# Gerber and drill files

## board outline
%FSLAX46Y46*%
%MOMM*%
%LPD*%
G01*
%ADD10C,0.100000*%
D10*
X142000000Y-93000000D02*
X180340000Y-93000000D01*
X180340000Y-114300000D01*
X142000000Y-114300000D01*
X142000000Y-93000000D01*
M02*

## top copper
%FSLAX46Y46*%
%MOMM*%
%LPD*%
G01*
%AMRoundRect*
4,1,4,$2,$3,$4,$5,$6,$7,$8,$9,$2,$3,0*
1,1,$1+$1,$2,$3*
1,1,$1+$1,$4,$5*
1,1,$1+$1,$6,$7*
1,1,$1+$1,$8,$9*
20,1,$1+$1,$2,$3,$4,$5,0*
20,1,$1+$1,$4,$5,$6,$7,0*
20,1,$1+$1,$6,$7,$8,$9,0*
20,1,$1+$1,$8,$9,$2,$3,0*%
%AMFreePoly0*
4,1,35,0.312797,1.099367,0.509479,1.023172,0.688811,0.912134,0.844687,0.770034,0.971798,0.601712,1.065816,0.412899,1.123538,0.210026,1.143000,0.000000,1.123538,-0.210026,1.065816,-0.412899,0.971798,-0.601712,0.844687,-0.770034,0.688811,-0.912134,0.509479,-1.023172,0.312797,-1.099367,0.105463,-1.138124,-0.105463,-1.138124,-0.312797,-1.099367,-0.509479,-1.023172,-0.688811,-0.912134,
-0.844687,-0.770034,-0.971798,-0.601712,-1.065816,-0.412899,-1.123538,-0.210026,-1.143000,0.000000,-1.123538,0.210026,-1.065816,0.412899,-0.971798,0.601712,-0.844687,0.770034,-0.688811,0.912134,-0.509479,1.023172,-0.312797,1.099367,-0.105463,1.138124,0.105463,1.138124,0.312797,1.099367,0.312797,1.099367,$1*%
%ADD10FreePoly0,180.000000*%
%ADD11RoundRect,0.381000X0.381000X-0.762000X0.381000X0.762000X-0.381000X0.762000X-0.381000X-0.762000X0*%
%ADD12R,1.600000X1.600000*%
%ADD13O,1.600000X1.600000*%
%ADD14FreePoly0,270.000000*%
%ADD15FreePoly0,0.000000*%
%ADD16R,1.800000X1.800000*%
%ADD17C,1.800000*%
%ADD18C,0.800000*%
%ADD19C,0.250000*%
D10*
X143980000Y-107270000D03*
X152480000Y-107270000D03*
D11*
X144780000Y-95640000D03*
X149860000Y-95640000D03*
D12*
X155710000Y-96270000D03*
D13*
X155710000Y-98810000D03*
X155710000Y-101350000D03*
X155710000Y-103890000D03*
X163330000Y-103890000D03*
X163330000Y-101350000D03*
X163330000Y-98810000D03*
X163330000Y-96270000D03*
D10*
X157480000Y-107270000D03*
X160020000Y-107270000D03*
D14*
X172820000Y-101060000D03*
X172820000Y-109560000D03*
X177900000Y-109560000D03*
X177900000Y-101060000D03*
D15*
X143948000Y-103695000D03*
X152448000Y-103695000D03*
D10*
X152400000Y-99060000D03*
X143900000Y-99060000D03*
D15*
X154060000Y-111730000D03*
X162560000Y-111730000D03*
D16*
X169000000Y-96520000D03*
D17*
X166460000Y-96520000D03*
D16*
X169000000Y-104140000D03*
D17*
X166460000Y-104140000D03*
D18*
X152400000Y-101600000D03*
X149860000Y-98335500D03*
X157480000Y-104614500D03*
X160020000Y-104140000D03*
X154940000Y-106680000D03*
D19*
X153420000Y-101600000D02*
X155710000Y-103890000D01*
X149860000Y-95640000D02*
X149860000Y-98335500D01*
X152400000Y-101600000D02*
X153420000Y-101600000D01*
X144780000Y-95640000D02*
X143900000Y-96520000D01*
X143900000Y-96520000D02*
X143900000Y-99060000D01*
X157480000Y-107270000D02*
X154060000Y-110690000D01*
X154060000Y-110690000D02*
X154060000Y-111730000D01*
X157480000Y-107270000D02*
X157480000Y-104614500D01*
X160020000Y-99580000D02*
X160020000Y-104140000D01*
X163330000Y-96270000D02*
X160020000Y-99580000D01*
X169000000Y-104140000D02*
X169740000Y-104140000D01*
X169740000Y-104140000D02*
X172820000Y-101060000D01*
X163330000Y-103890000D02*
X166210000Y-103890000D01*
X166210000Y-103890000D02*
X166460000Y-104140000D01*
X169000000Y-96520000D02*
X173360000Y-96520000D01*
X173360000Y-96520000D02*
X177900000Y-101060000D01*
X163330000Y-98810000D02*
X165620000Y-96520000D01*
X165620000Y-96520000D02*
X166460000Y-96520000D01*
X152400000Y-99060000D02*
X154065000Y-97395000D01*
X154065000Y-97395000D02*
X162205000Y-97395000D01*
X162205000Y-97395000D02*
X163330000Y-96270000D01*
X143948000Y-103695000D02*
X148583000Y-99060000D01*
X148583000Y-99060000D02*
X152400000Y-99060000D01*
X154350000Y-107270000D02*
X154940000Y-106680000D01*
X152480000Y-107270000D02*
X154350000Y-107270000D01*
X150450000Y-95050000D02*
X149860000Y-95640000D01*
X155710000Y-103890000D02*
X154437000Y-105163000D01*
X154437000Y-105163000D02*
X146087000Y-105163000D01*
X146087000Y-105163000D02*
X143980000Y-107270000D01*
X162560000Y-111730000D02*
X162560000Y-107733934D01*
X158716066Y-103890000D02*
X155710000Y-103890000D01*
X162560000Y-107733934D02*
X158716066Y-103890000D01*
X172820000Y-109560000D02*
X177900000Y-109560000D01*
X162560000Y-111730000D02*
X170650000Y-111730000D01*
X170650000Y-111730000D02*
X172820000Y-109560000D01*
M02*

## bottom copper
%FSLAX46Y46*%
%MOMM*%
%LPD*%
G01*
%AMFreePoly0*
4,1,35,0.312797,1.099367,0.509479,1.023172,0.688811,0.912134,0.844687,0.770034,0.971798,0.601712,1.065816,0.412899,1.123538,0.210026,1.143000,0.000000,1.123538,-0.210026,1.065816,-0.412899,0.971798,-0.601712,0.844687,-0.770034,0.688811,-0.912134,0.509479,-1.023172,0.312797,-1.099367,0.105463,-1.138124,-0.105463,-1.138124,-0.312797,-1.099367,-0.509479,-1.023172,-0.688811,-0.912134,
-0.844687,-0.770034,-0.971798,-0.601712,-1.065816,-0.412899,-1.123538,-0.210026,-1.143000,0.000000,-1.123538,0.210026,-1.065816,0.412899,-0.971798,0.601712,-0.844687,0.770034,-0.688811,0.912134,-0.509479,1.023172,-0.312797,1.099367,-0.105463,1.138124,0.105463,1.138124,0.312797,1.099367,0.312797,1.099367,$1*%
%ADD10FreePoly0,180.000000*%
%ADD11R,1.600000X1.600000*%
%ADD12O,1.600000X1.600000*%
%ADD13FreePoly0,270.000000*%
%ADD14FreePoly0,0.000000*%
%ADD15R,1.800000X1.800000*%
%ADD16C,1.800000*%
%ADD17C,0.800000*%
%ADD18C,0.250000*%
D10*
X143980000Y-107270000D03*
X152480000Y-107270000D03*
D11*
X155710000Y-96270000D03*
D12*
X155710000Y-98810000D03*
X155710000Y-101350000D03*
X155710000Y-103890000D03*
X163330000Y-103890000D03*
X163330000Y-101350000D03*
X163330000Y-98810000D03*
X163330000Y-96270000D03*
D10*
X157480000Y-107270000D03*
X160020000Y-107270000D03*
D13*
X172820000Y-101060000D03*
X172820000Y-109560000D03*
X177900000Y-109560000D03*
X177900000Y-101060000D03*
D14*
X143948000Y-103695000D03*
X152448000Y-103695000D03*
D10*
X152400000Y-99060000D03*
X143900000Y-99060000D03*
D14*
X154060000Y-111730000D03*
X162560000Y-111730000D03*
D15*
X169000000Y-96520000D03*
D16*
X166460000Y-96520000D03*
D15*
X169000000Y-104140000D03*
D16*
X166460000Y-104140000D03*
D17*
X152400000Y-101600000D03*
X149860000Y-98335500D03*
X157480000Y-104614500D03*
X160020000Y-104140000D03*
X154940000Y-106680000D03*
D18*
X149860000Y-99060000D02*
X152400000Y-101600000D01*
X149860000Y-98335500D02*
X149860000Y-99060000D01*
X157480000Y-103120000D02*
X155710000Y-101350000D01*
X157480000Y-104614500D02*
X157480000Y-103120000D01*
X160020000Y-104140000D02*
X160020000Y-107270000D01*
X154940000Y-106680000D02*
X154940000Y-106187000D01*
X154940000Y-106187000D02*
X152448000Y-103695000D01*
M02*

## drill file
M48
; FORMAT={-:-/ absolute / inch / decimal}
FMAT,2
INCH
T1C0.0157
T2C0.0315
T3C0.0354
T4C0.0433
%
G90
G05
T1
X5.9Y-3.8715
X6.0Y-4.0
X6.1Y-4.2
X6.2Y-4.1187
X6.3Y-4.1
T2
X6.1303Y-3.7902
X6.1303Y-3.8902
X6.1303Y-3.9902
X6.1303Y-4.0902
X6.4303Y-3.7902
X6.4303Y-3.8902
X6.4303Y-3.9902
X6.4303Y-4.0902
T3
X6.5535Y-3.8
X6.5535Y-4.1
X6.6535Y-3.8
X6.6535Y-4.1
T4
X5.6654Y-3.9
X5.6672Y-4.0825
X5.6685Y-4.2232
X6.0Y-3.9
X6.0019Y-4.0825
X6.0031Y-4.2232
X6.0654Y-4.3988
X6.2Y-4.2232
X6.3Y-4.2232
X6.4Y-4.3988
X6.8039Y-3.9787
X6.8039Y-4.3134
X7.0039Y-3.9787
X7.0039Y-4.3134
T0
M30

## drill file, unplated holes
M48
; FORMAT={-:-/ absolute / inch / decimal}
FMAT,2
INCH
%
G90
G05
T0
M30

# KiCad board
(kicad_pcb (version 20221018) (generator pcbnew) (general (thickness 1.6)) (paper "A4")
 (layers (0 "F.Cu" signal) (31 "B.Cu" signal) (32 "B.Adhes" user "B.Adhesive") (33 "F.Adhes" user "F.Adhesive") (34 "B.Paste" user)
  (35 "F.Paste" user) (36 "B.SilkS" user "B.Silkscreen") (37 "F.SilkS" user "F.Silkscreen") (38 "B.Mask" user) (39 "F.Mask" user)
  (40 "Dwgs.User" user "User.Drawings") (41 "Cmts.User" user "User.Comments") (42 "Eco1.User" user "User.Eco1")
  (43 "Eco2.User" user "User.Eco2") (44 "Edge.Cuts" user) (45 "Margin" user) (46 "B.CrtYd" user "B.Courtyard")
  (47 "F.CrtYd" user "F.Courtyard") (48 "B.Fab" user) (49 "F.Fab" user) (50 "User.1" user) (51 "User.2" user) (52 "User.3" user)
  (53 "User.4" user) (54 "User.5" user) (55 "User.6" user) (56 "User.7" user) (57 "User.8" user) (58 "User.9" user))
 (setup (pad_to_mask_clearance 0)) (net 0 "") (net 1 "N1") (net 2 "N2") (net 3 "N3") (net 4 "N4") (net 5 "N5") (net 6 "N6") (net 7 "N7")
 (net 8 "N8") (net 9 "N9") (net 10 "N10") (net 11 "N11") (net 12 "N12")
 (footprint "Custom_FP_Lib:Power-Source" (layer "F.Cu") (at 147.32 98.18 90)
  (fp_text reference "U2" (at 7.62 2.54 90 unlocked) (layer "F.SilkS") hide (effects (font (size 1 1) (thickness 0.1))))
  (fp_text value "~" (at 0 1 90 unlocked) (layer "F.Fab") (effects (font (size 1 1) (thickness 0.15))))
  (pad "1" smd roundrect (at 2.54 -2.54 90) (size 2.286 1.524) (layers "F.Cu" "F.Paste" "F.Mask") (roundrect_rratio 0.25) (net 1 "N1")
   (thermal_bridge_angle 45))
  (pad "2" smd roundrect (at 2.54 2.54 90) (size 2.286 1.524) (layers "F.Cu" "F.Paste" "F.Mask") (roundrect_rratio 0.25) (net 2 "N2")
   (thermal_bridge_angle 45)))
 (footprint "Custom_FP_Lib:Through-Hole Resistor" (layer "F.Cu") (at 143.628 104.965)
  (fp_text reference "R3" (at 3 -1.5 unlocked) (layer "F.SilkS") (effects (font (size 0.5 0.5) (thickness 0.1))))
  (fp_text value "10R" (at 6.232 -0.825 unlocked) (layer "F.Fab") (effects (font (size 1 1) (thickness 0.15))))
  (pad "1" thru_hole custom (at 0.32 -1.27) (size 2.286 2.286) (drill 1.1) (layers "*.Cu" "*.Mask") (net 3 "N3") (thermal_bridge_angle 45)
   (options (clearance outline) (anchor circle)) (primitives))
  (pad "2" thru_hole custom (at 8.82 -1.27) (size 2.286 2.286) (drill 1.1) (layers "*.Cu" "*.Mask") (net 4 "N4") (thermal_bridge_angle 45)
   (options (clearance outline) (anchor circle)) (primitives)))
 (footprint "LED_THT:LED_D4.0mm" (layer "F.Cu") (at 169 104.14 180)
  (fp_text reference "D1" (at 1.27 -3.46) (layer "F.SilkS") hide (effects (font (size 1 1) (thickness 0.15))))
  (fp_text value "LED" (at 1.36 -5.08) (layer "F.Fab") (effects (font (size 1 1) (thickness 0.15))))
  (pad "1" thru_hole rect (at 0 0 180) (size 1.8 1.8) (drill 0.9) (layers "*.Cu" "*.Mask") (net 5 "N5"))
  (pad "2" thru_hole circle (at 2.54 0 180) (size 1.8 1.8) (drill 0.9) (layers "*.Cu" "*.Mask") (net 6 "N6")))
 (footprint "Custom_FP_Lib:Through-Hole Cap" (layer "F.Cu") (at 160.02 106 180)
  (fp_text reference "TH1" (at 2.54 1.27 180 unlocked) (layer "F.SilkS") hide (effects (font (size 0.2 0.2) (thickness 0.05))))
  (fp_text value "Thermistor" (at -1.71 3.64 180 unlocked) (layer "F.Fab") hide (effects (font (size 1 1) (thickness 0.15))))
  (pad "1" thru_hole custom (at 0 -1.27 180) (size 2.286 2.286) (drill 1.1) (layers "*.Cu" "*.Mask") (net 3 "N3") (thermal_bridge_angle 45)
   (options (clearance outline) (anchor circle)) (primitives))
  (pad "2" thru_hole custom (at 2.54 -1.27 180) (size 2.286 2.286) (drill 1.1) (layers "*.Cu" "*.Mask") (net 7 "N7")
   (thermal_bridge_angle 45) (options (clearance outline) (anchor circle)) (primitives)))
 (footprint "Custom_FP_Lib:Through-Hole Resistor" (layer "F.Cu") (at 176.63 100.74 -90)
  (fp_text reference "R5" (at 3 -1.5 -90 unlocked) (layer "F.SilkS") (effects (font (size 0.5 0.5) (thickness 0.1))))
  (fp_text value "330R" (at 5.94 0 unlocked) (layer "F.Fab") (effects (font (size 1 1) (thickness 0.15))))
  (pad "1" thru_hole custom (at 0.32 -1.27 270) (size 2.286 2.286) (drill 1.1) (layers "*.Cu" "*.Mask") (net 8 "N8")
   (thermal_bridge_angle 45) (options (clearance outline) (anchor circle)) (primitives))
  (pad "2" thru_hole custom (at 8.82 -1.27 270) (size 2.286 2.286) (drill 1.1) (layers "*.Cu" "*.Mask") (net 2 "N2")
   (thermal_bridge_angle 45) (options (clearance outline) (anchor circle)) (primitives)))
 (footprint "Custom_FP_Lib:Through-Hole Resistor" (layer "F.Cu") (at 152.8 106 180)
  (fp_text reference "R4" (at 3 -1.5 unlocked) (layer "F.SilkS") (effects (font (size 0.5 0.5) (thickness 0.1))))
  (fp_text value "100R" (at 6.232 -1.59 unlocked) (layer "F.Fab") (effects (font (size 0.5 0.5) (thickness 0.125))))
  (pad "1" thru_hole custom (at 0.32 -1.27 180) (size 2.286 2.286) (drill 1.1) (layers "*.Cu" "*.Mask") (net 4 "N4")
   (thermal_bridge_angle 45) (options (clearance outline) (anchor circle)) (primitives))
  (pad "2" thru_hole custom (at 8.82 -1.27 180) (size 2.286 2.286) (drill 1.1) (layers "*.Cu" "*.Mask") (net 2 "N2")
   (thermal_bridge_angle 45) (options (clearance outline) (anchor circle)) (primitives)))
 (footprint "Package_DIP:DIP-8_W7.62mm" (layer "F.Cu") (at 155.71 96.27)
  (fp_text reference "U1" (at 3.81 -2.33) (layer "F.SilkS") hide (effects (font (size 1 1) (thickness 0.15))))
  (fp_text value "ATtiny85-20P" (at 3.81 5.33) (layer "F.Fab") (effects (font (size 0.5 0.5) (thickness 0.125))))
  (pad "1" thru_hole rect (at 0 0) (size 1.6 1.6) (drill 0.8) (layers "*.Cu" "*.Mask") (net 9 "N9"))
  (pad "2" thru_hole oval (at 0 2.54) (size 1.6 1.6) (drill 0.8) (layers "*.Cu" "*.Mask") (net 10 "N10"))
  (pad "3" thru_hole oval (at 0 5.08) (size 1.6 1.6) (drill 0.8) (layers "*.Cu" "*.Mask") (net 7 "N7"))
  (pad "4" thru_hole oval (at 0 7.62) (size 1.6 1.6) (drill 0.8) (layers "*.Cu" "*.Mask") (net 2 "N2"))
  (pad "5" thru_hole oval (at 7.62 7.62) (size 1.6 1.6) (drill 0.8) (layers "*.Cu" "*.Mask") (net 6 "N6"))
  (pad "6" thru_hole oval (at 7.62 5.08) (size 1.6 1.6) (drill 0.8) (layers "*.Cu" "*.Mask") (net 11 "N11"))
  (pad "7" thru_hole oval (at 7.62 2.54) (size 1.6 1.6) (drill 0.8) (layers "*.Cu" "*.Mask") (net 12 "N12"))
  (pad "8" thru_hole oval (at 7.62 0) (size 1.6 1.6) (drill 0.8) (layers "*.Cu" "*.Mask") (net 3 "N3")))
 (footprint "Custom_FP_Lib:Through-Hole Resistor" (layer "F.Cu") (at 152.72 97.79 180)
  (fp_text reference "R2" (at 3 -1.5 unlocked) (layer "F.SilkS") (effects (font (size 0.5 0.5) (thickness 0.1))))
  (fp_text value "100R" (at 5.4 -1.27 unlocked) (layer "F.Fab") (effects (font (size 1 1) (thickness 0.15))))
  (pad "1" thru_hole custom (at 0.32 -1.27 180) (size 2.286 2.286) (drill 1.1) (layers "*.Cu" "*.Mask") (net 3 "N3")
   (thermal_bridge_angle 45) (options (clearance outline) (anchor circle)) (primitives))
  (pad "2" thru_hole custom (at 8.82 -1.27 180) (size 2.286 2.286) (drill 1.1) (layers "*.Cu" "*.Mask") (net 1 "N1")
   (thermal_bridge_angle 45) (options (clearance outline) (anchor circle)) (primitives)))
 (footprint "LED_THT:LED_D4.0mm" (layer "F.Cu") (at 169 96.52 180)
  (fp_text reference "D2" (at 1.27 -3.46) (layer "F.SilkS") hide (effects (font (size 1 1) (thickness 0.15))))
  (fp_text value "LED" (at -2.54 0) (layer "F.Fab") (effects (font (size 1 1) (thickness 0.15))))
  (pad "1" thru_hole rect (at 0 0 180) (size 1.8 1.8) (drill 0.9) (layers "*.Cu" "*.Mask") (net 8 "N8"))
  (pad "2" thru_hole circle (at 2.54 0 180) (size 1.8 1.8) (drill 0.9) (layers "*.Cu" "*.Mask") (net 12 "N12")))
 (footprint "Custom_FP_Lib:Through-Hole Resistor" (layer "F.Cu") (at 171.55 100.74 -90)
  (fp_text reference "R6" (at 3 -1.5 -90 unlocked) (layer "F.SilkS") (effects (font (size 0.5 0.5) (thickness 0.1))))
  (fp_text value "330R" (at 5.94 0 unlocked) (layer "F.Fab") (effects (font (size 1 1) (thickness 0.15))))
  (pad "1" thru_hole custom (at 0.32 -1.27 270) (size 2.286 2.286) (drill 1.1) (layers "*.Cu" "*.Mask") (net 5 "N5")
   (thermal_bridge_angle 45) (options (clearance outline) (anchor circle)) (primitives))
  (pad "2" thru_hole custom (at 8.82 -1.27 270) (size 2.286 2.286) (drill 1.1) (layers "*.Cu" "*.Mask") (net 2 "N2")
   (thermal_bridge_angle 45) (options (clearance outline) (anchor circle)) (primitives)))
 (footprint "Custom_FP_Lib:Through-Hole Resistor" (layer "F.Cu") (at 153.74 113)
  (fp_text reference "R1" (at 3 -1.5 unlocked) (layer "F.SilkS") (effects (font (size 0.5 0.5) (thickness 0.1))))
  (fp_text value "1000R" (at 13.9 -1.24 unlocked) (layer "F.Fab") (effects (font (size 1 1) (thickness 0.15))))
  (pad "1" thru_hole custom (at 0.32 -1.27) (size 2.286 2.286) (drill 1.1) (layers "*.Cu" "*.Mask") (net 7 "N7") (thermal_bridge_angle 45)
   (options (clearance outline) (anchor circle)) (primitives))
  (pad "2" thru_hole custom (at 8.82 -1.27) (size 2.286 2.286) (drill 1.1) (layers "*.Cu" "*.Mask") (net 2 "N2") (thermal_bridge_angle 45)
   (options (clearance outline) (anchor circle)) (primitives)))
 (gr_rect (start 142 93) (end 180.34 114.3) (stroke (width 0.1) (type default)) (fill none) (layer "Edge.Cuts"))
 (segment (start 169.74 104.14) (end 172.82 101.06) (width 0.25) (layer "F.Cu") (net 5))
 (segment (start 169 104.14) (end 169.74 104.14) (width 0.25) (layer "F.Cu") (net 5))
 (segment (start 166.21 103.89) (end 166.46 104.14) (width 0.25) (layer "F.Cu") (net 6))
 (segment (start 163.33 103.89) (end 166.21 103.89) (width 0.25) (layer "F.Cu") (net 6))
 (segment (start 163.33 98.81) (end 165.62 96.52) (width 0.25) (layer "F.Cu") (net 12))
 (segment (start 165.62 96.52) (end 166.46 96.52) (width 0.25) (layer "F.Cu") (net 12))
 (segment (start 154.06 110.69) (end 154.06 111.73) (width 0.25) (layer "F.Cu") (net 7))
 (segment (start 157.48 107.27) (end 154.06 110.69) (width 0.25) (layer "F.Cu") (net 7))
 (segment (start 157.48 107.27) (end 157.48 104.6145) (width 0.25) (layer "F.Cu") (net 7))
 (via (at 157.48 104.6145) (size 0.8) (drill 0.4) (layers "F.Cu" "B.Cu") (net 7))
 (segment (start 157.48 104.6145) (end 157.48 103.12) (width 0.25) (layer "B.Cu") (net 7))
 (segment (start 157.48 103.12) (end 155.71 101.35) (width 0.25) (layer "B.Cu") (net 7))
 (segment (start 162.205 97.395) (end 163.33 96.27) (width 0.25) (layer "F.Cu") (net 3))
 (segment (start 152.4 99.06) (end 154.065 97.395) (width 0.25) (layer "F.Cu") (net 3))
 (segment (start 148.583 99.06) (end 152.4 99.06) (width 0.25) (layer "F.Cu") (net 3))
 (segment (start 160.02 99.58) (end 160.02 104.14) (width 0.25) (layer "F.Cu") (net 3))
 (segment (start 163.33 96.27) (end 160.02 99.58) (width 0.25) (layer "F.Cu") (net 3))
 (segment (start 143.948 103.695) (end 148.583 99.06) (width 0.25) (layer "F.Cu") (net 3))
 (segment (start 154.065 97.395) (end 162.205 97.395) (width 0.25) (layer "F.Cu") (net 3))
 (via (at 160.02 104.14) (size 0.8) (drill 0.4) (layers "F.Cu" "B.Cu") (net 3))
 (segment (start 160.02 104.14) (end 160.02 107.27) (width 0.25) (layer "B.Cu") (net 3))
 (segment (start 143.9 96.52) (end 143.9 99.06) (width 0.25) (layer "F.Cu") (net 1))
 (segment (start 144.78 95.64) (end 143.9 96.52) (width 0.25) (layer "F.Cu") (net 1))
 (segment (start 152.48 107.27) (end 154.35 107.27) (width 0.25) (layer "F.Cu") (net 4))
 (segment (start 154.35 107.27) (end 154.94 106.68) (width 0.25) (layer "F.Cu") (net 4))
 (via (at 154.94 106.68) (size 0.8) (drill 0.4) (layers "F.Cu" "B.Cu") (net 4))
 (segment (start 154.94 106.187) (end 152.448 103.695) (width 0.25) (layer "B.Cu") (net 4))
 (segment (start 154.94 106.68) (end 154.94 106.187) (width 0.25) (layer "B.Cu") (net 4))
 (segment (start 173.36 96.52) (end 177.9 101.06) (width 0.25) (layer "F.Cu") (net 8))
 (segment (start 169 96.52) (end 173.36 96.52) (width 0.25) (layer "F.Cu") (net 8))
 (segment (start 146.087 105.163) (end 143.98 107.27) (width 0.25) (layer "F.Cu") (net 2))
 (segment (start 153.42 101.6) (end 155.71 103.89) (width 0.25) (layer "F.Cu") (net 2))
 (segment (start 162.56 107.733934) (end 158.716066 103.89) (width 0.25) (layer "F.Cu") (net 2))
 (segment (start 152.4 101.6) (end 153.42 101.6) (width 0.25) (layer "F.Cu") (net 2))
 (segment (start 162.56 111.73) (end 162.56 107.733934) (width 0.25) (layer "F.Cu") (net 2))
 (segment (start 155.71 103.89) (end 154.437 105.163) (width 0.25) (layer "F.Cu") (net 2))
 (segment (start 172.82 109.56) (end 177.9 109.56) (width 0.25) (layer "F.Cu") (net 2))
 (segment (start 149.86 95.64) (end 149.86 98.3355) (width 0.25) (layer "F.Cu") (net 2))
 (segment (start 170.65 111.73) (end 172.82 109.56) (width 0.25) (layer "F.Cu") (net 2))
 (segment (start 162.56 111.73) (end 170.65 111.73) (width 0.25) (layer "F.Cu") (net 2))
 (segment (start 150.45 95.05) (end 149.86 95.64) (width 0.25) (layer "F.Cu") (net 2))
 (segment (start 154.437 105.163) (end 146.087 105.163) (width 0.25) (layer "F.Cu") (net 2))
 (segment (start 158.716066 103.89) (end 155.71 103.89) (width 0.25) (layer "F.Cu") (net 2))
 (via (at 152.4 101.6) (size 0.8) (drill 0.4) (layers "F.Cu" "B.Cu") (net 2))
 (via (at 149.86 98.3355) (size 0.8) (drill 0.4) (layers "F.Cu" "B.Cu") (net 2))
 (segment (start 149.86 98.3355) (end 149.86 99.06) (width 0.25) (layer "B.Cu") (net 2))
 (segment (start 149.86 99.06) (end 152.4 101.6) (width 0.25) (layer "B.Cu") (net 2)))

